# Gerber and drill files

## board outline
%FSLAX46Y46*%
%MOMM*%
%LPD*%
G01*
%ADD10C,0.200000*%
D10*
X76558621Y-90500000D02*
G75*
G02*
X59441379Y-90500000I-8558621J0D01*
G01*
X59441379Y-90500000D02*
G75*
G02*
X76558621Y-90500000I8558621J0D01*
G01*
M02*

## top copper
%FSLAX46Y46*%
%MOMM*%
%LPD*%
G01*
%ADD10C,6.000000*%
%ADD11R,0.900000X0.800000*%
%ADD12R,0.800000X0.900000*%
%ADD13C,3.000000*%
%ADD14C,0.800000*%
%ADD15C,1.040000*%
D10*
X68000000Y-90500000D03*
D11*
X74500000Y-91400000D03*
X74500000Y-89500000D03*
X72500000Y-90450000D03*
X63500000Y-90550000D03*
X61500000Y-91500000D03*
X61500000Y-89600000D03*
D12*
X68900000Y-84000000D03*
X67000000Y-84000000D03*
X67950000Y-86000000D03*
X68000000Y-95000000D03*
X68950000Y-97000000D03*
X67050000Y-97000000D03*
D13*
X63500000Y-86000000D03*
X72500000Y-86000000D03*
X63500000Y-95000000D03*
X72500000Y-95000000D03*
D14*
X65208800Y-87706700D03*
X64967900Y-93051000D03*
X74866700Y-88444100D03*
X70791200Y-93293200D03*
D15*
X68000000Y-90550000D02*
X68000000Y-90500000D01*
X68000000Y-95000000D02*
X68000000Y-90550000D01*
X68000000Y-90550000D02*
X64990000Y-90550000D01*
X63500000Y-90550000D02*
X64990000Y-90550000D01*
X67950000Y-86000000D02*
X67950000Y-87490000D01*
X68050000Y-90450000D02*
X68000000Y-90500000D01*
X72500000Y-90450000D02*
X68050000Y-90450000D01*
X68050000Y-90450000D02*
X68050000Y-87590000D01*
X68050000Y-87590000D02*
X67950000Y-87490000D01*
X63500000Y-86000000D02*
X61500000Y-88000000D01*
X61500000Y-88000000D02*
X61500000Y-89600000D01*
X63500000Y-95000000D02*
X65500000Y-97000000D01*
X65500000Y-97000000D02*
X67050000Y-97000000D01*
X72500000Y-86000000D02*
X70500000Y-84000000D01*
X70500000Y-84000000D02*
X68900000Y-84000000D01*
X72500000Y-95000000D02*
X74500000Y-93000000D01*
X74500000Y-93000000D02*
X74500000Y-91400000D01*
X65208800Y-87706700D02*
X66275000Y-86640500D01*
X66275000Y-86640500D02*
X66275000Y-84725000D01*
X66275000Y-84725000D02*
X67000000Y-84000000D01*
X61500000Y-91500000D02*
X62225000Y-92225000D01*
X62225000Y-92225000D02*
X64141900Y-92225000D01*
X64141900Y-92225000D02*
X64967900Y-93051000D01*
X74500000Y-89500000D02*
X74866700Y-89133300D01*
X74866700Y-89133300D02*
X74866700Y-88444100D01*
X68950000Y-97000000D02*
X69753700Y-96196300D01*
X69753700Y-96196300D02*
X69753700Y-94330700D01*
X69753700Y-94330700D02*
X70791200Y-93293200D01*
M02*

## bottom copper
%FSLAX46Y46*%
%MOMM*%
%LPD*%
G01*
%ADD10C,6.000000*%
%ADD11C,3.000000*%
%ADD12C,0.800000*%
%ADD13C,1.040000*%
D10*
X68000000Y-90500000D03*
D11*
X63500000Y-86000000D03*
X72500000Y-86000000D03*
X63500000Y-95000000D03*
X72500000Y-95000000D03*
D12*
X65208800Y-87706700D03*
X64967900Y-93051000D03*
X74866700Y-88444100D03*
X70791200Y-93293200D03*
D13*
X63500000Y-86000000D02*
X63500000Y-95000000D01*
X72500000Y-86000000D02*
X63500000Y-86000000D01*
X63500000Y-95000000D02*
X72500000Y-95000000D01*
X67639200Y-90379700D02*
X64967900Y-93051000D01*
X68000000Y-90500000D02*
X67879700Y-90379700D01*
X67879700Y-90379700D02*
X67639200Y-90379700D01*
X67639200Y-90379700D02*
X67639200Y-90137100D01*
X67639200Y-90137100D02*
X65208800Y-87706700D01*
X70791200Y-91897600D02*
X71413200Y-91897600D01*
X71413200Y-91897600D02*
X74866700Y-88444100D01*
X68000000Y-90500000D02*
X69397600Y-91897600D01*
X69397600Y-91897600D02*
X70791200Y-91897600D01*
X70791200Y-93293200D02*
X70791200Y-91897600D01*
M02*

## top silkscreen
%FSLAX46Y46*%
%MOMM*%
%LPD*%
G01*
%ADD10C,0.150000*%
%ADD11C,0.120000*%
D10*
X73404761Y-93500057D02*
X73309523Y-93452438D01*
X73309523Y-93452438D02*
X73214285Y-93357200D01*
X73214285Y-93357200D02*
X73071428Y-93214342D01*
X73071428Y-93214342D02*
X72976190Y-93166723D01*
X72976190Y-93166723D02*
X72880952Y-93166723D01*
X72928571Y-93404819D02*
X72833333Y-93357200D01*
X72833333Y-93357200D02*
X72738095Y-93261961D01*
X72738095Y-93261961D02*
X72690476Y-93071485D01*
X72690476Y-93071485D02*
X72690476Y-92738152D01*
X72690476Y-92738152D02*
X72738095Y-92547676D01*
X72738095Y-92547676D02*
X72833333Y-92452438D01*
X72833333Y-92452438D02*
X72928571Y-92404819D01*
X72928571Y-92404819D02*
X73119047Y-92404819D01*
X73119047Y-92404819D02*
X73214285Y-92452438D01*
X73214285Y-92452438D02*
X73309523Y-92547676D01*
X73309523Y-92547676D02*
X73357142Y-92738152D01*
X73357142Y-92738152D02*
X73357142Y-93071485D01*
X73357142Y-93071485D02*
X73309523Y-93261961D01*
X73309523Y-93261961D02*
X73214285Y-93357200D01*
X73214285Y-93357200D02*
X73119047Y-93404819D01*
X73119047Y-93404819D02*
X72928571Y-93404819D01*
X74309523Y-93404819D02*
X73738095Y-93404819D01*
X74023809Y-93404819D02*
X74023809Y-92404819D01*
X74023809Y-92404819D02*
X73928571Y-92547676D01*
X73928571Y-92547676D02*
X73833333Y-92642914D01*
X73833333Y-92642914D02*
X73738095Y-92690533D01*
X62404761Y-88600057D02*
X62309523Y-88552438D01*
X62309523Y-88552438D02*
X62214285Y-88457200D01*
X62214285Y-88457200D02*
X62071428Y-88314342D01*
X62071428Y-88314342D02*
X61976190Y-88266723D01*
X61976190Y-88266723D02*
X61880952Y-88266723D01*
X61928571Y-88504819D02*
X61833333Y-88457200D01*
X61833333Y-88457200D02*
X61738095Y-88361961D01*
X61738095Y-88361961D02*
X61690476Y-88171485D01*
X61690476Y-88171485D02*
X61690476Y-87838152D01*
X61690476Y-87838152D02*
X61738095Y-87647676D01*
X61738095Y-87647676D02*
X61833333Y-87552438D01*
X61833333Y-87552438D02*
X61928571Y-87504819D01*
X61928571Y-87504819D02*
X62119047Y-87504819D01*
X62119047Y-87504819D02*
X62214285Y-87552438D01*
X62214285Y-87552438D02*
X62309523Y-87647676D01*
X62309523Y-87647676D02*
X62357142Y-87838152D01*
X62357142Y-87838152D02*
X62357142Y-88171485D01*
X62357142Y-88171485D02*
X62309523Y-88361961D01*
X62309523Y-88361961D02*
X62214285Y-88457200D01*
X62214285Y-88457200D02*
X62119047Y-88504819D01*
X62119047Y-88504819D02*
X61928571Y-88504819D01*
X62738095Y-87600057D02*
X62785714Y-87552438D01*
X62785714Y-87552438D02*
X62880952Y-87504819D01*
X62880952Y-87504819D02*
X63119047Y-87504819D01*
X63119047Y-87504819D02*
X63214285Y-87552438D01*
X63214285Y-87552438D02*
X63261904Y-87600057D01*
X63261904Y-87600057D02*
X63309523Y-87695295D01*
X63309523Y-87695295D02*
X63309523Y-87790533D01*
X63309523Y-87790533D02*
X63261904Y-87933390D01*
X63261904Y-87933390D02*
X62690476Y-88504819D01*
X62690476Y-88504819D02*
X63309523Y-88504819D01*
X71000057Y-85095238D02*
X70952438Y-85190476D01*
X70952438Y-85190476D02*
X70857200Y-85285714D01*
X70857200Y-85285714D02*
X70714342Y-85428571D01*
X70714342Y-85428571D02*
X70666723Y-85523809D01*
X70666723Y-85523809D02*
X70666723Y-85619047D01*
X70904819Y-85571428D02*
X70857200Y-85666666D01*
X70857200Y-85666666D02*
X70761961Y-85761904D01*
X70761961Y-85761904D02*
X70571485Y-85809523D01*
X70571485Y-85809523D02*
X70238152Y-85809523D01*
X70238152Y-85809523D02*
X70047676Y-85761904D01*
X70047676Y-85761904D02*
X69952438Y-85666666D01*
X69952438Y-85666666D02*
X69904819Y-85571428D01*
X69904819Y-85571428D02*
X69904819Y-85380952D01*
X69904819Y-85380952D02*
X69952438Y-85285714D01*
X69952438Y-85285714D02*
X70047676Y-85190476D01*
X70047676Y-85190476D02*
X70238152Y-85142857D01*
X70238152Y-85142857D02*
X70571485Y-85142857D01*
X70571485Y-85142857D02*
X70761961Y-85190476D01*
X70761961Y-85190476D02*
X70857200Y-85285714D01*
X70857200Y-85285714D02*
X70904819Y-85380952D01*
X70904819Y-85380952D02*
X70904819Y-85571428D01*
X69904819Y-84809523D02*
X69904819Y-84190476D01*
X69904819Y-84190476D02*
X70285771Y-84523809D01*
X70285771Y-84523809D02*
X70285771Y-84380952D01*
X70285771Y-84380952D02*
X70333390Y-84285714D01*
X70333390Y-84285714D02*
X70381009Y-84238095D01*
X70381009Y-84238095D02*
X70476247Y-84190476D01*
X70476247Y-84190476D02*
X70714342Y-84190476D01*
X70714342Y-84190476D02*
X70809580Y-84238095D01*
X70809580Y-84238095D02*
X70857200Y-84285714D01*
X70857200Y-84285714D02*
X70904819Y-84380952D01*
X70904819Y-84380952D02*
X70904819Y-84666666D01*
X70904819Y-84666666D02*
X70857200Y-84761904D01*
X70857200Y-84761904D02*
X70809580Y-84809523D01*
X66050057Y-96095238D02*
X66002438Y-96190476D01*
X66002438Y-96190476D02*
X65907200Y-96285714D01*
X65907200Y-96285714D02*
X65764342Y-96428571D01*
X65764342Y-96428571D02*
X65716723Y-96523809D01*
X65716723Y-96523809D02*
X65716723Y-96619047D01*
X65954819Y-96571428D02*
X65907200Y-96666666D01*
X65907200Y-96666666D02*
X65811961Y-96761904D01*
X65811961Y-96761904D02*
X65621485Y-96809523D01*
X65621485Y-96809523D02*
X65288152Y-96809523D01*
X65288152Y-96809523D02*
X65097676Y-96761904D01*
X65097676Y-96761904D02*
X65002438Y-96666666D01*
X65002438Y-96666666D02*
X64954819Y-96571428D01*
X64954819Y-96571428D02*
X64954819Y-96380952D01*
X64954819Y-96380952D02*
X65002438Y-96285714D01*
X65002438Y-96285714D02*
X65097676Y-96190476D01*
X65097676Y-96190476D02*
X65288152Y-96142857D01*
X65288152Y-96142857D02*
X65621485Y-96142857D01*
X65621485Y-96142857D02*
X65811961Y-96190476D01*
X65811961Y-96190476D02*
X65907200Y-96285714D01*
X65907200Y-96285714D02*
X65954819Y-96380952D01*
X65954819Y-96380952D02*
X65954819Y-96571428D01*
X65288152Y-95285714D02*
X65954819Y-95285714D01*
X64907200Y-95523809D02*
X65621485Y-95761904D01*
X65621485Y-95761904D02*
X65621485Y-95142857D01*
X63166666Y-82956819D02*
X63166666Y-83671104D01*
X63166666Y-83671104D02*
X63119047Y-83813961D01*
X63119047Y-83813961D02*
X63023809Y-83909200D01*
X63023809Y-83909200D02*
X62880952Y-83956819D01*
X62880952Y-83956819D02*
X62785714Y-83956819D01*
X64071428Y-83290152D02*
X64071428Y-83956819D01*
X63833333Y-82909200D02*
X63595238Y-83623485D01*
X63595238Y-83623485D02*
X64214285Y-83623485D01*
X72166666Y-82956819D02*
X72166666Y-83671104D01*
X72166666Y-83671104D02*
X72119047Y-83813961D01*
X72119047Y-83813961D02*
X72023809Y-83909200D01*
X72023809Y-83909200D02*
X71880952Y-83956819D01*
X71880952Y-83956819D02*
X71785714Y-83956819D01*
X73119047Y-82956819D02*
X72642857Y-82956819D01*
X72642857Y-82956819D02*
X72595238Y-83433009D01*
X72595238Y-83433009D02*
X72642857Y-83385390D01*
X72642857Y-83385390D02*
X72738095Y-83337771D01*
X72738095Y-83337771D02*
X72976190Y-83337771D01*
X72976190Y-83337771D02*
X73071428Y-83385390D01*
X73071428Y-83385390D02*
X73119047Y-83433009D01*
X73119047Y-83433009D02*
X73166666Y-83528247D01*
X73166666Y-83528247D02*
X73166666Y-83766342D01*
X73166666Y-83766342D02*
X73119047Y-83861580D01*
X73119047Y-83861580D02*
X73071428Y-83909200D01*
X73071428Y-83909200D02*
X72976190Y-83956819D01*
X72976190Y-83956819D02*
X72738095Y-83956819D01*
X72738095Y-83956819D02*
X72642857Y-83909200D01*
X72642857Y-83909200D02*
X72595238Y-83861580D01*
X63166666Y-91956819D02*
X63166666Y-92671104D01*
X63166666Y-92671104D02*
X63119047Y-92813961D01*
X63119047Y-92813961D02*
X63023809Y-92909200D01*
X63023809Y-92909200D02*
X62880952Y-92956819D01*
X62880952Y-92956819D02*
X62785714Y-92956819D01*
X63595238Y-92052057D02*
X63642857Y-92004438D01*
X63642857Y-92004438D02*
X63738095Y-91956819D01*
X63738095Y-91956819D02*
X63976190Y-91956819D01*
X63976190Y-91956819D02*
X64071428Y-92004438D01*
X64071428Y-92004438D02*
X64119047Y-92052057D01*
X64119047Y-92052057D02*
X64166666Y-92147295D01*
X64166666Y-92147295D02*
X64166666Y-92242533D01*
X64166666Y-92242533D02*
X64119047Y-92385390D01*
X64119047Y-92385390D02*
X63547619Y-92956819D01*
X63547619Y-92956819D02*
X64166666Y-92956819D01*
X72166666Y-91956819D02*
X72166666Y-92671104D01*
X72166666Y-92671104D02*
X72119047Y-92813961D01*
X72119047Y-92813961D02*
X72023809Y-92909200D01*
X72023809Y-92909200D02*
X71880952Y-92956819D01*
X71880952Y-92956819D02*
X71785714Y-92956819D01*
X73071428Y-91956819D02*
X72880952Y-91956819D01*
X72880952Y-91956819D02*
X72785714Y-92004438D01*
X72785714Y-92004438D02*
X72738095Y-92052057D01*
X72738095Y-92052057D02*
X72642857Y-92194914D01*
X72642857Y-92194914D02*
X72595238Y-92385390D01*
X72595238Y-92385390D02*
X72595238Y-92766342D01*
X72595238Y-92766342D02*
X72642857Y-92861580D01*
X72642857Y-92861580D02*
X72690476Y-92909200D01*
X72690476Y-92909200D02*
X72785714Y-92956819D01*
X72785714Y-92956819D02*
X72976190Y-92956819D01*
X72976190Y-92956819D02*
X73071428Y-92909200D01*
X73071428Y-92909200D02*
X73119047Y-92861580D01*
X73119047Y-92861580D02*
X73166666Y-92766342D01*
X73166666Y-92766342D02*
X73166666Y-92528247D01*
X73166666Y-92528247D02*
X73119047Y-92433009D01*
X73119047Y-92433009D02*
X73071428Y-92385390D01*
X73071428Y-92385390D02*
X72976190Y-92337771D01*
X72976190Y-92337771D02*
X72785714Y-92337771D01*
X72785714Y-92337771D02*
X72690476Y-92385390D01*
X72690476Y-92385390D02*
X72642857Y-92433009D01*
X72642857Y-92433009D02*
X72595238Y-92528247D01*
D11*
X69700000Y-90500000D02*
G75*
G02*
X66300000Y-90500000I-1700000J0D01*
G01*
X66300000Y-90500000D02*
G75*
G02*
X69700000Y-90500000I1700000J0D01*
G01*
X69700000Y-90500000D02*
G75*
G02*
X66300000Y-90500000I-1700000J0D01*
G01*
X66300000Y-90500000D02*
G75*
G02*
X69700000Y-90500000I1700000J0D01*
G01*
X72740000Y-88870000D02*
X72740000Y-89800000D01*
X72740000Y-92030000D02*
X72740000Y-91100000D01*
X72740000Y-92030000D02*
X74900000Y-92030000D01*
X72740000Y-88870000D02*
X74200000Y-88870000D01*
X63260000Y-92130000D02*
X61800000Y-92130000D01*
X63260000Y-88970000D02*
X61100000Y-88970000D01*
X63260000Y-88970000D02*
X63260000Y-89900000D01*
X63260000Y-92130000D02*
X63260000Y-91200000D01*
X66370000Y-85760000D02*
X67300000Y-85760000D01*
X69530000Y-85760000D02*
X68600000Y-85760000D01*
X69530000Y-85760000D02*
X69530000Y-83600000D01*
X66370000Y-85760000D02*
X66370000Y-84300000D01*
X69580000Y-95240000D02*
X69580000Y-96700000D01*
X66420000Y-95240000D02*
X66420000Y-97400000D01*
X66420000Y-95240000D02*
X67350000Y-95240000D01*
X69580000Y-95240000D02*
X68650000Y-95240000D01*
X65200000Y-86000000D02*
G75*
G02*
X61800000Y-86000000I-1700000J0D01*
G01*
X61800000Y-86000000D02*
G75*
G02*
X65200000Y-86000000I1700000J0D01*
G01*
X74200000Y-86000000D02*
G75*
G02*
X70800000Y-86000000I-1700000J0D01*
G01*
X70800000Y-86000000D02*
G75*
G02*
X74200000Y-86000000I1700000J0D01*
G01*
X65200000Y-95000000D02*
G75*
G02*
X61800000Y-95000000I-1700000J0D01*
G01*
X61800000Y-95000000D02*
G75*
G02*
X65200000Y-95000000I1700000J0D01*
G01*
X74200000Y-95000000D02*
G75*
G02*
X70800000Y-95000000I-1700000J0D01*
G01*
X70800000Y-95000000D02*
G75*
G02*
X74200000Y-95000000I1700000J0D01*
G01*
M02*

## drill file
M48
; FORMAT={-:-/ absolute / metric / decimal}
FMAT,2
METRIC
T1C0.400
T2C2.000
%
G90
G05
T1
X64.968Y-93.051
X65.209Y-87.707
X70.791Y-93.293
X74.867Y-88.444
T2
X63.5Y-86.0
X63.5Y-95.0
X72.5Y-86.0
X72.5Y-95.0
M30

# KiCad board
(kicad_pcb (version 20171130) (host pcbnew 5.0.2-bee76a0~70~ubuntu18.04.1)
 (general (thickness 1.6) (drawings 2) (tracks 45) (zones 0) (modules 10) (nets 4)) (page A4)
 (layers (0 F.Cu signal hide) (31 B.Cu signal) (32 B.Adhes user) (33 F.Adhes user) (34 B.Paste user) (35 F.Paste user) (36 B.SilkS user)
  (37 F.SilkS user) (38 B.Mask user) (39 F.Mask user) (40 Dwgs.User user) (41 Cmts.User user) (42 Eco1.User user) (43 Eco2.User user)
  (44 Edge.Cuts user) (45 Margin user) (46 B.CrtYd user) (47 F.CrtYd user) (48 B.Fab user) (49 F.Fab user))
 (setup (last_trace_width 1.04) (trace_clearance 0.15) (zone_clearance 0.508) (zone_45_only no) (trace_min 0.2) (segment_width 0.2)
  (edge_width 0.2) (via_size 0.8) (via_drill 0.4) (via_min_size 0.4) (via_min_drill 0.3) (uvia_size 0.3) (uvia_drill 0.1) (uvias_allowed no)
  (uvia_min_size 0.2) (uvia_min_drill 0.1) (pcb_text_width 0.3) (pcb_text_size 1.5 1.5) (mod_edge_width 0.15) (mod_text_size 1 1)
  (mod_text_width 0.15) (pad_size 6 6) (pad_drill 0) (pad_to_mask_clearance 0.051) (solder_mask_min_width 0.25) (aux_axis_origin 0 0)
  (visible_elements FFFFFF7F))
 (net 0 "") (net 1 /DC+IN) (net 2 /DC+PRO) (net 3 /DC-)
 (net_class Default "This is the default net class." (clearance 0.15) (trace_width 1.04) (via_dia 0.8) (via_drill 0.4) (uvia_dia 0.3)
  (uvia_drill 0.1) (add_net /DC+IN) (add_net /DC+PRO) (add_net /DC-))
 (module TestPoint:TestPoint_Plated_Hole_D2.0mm (layer F.Cu) (at 68 90.5)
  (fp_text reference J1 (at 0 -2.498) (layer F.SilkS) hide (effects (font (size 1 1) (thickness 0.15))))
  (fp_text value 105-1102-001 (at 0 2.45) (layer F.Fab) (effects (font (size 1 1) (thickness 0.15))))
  (fp_circle (center 0 0) (end 0 -1.7) (layer F.SilkS) (width 0.12))
  (pad 1 smd circle (at 0 0) (size 6 6) (layers F.Cu F.Paste F.Mask) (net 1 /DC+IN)))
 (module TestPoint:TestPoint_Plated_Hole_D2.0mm (layer F.Cu) (at 68 90.5)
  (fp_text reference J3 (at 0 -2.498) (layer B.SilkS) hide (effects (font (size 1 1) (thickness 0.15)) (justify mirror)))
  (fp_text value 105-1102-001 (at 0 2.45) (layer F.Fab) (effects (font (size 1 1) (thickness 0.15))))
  (fp_circle (center 0 0) (end 0 -1.7) (layer F.SilkS) (width 0.12))
  (pad 1 smd circle (at 0 0) (size 6 6) (layers B.Cu F.Paste F.Mask) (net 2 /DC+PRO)))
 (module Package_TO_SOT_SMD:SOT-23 (layer F.Cu) (at 73.5 90.45 180)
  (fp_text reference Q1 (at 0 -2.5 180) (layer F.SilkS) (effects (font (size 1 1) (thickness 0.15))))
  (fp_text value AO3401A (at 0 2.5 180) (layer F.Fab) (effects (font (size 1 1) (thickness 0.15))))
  (fp_line (start 0.76 1.58) (end 0.76 0.65) (layer F.SilkS) (width 0.12))
  (fp_line (start 0.76 -1.58) (end 0.76 -0.65) (layer F.SilkS) (width 0.12))
  (fp_line (start 0.76 -1.58) (end -1.4 -1.58) (layer F.SilkS) (width 0.12))
  (fp_line (start 0.76 1.58) (end -0.7 1.58) (layer F.SilkS) (width 0.12))
  (pad 1 smd rect (at -1 -0.95 180) (size 0.9 0.8) (layers F.Cu F.Paste F.Mask) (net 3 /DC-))
  (pad 2 smd rect (at -1 0.95 180) (size 0.9 0.8) (layers F.Cu F.Paste F.Mask) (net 2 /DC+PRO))
  (pad 3 smd rect (at 1 0 180) (size 0.9 0.8) (layers F.Cu F.Paste F.Mask) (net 1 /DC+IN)))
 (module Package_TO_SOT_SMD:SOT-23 (layer F.Cu) (at 62.5 90.55)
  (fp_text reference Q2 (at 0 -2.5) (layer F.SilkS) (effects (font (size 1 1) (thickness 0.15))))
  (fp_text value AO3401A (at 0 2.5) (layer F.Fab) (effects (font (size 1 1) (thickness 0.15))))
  (fp_line (start 0.76 1.58) (end -0.7 1.58) (layer F.SilkS) (width 0.12))
  (fp_line (start 0.76 -1.58) (end -1.4 -1.58) (layer F.SilkS) (width 0.12))
  (fp_line (start 0.76 -1.58) (end 0.76 -0.65) (layer F.SilkS) (width 0.12))
  (fp_line (start 0.76 1.58) (end 0.76 0.65) (layer F.SilkS) (width 0.12))
  (pad 3 smd rect (at 1 0) (size 0.9 0.8) (layers F.Cu F.Paste F.Mask) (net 1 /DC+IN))
  (pad 2 smd rect (at -1 0.95) (size 0.9 0.8) (layers F.Cu F.Paste F.Mask) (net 2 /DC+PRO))
  (pad 1 smd rect (at -1 -0.95) (size 0.9 0.8) (layers F.Cu F.Paste F.Mask) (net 3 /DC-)))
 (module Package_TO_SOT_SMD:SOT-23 (layer F.Cu) (at 67.95 85 270)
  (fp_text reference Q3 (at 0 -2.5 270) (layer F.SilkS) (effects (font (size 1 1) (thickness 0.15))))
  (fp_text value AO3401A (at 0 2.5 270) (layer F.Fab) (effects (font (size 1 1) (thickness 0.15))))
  (fp_line (start 0.76 1.58) (end 0.76 0.65) (layer F.SilkS) (width 0.12))
  (fp_line (start 0.76 -1.58) (end 0.76 -0.65) (layer F.SilkS) (width 0.12))
  (fp_line (start 0.76 -1.58) (end -1.4 -1.58) (layer F.SilkS) (width 0.12))
  (fp_line (start 0.76 1.58) (end -0.7 1.58) (layer F.SilkS) (width 0.12))
  (pad 1 smd rect (at -1 -0.95 270) (size 0.9 0.8) (layers F.Cu F.Paste F.Mask) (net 3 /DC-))
  (pad 2 smd rect (at -1 0.95 270) (size 0.9 0.8) (layers F.Cu F.Paste F.Mask) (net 2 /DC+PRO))
  (pad 3 smd rect (at 1 0 270) (size 0.9 0.8) (layers F.Cu F.Paste F.Mask) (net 1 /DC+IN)))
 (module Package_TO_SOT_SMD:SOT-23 (layer F.Cu) (at 68 96 90)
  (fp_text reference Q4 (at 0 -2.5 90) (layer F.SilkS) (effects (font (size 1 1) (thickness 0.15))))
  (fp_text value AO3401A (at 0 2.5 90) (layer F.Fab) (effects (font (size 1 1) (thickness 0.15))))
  (fp_line (start 0.76 1.58) (end -0.7 1.58) (layer F.SilkS) (width 0.12))
  (fp_line (start 0.76 -1.58) (end -1.4 -1.58) (layer F.SilkS) (width 0.12))
  (fp_line (start 0.76 -1.58) (end 0.76 -0.65) (layer F.SilkS) (width 0.12))
  (fp_line (start 0.76 1.58) (end 0.76 0.65) (layer F.SilkS) (width 0.12))
  (pad 3 smd rect (at 1 0 90) (size 0.9 0.8) (layers F.Cu F.Paste F.Mask) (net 1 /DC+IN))
  (pad 2 smd rect (at -1 0.95 90) (size 0.9 0.8) (layers F.Cu F.Paste F.Mask) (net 2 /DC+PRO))
  (pad 1 smd rect (at -1 -0.95 90) (size 0.9 0.8) (layers F.Cu F.Paste F.Mask) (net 3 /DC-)))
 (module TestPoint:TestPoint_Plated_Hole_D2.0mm (layer F.Cu) (at 63.5 86)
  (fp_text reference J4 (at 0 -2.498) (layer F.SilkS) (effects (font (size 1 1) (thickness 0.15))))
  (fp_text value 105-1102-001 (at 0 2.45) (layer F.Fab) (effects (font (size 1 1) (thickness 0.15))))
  (fp_circle (center 0 0) (end 0 -1.7) (layer F.SilkS) (width 0.12))
  (pad 1 thru_hole circle (at 0 0) (size 3 3) (drill 2) (layers *.Cu *.Mask) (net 3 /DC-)))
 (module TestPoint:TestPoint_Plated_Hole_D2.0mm (layer F.Cu) (at 72.5 86)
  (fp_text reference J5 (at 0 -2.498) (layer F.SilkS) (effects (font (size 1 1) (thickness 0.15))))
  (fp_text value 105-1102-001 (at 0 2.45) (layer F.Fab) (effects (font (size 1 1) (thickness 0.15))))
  (fp_circle (center 0 0) (end 0 -1.7) (layer F.SilkS) (width 0.12))
  (pad 1 thru_hole circle (at 0 0) (size 3 3) (drill 2) (layers *.Cu *.Mask) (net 3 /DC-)))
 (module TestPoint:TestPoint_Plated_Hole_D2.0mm (layer F.Cu) (at 63.5 95)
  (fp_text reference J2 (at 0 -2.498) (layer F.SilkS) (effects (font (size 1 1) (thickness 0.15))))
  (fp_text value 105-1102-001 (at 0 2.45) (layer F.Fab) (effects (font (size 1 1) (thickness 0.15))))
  (fp_circle (center 0 0) (end 0 -1.7) (layer F.SilkS) (width 0.12))
  (pad 1 thru_hole circle (at 0 0) (size 3 3) (drill 2) (layers *.Cu *.Mask) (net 3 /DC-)))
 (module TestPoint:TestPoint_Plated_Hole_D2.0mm (layer F.Cu) (at 72.5 95)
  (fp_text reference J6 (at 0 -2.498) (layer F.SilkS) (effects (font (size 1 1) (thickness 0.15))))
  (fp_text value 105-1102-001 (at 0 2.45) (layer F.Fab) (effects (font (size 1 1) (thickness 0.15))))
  (fp_circle (center 0 0) (end 0 -1.7) (layer F.SilkS) (width 0.12))
  (pad 1 thru_hole circle (at 0 0) (size 3 3) (drill 2) (layers *.Cu *.Mask) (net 3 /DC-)))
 (gr_circle (center 68 90.5) (end 76.558621 90.5) (layer Edge.Cuts) (width 0.2))
 (segment (start 68 90.55) (end 68 90.5) (width 1.04) (layer F.Cu) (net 1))
 (segment (start 68 95) (end 68 90.55) (width 1.04) (layer F.Cu) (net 1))
 (segment (start 68 90.55) (end 64.99 90.55) (width 1.04) (layer F.Cu) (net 1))
 (segment (start 63.5 90.55) (end 64.99 90.55) (width 1.04) (layer F.Cu) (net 1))
 (segment (start 67.95 86) (end 67.95 87.49) (width 1.04) (layer F.Cu) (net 1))
 (segment (start 68.05 90.45) (end 68 90.5) (width 1.04) (layer F.Cu) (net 1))
 (segment (start 72.5 90.45) (end 68.05 90.45) (width 1.04) (layer F.Cu) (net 1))
 (segment (start 68.05 90.45) (end 68.05 87.59) (width 1.04) (layer F.Cu) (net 1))
 (segment (start 68.05 87.59) (end 67.95 87.49) (width 1.04) (layer F.Cu) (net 1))
 (segment (start 63.5 86) (end 63.5 95) (width 1.04) (layer B.Cu) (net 3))
 (segment (start 72.5 86) (end 63.5 86) (width 1.04) (layer B.Cu) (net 3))
 (segment (start 63.5 95) (end 72.5 95) (width 1.04) (layer B.Cu) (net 3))
 (segment (start 63.5 86) (end 61.5 88) (width 1.04) (layer F.Cu) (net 3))
 (segment (start 61.5 88) (end 61.5 89.6) (width 1.04) (layer F.Cu) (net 3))
 (segment (start 63.5 95) (end 65.5 97) (width 1.04) (layer F.Cu) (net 3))
 (segment (start 65.5 97) (end 67.05 97) (width 1.04) (layer F.Cu) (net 3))
 (segment (start 72.5 86) (end 70.5 84) (width 1.04) (layer F.Cu) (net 3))
 (segment (start 70.5 84) (end 68.9 84) (width 1.04) (layer F.Cu) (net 3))
 (segment (start 72.5 95) (end 74.5 93) (width 1.04) (layer F.Cu) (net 3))
 (segment (start 74.5 93) (end 74.5 91.4) (width 1.04) (layer F.Cu) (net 3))
 (segment (start 67.6392 90.3797) (end 64.9679 93.051) (width 1.04) (layer B.Cu) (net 2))
 (segment (start 68 90.5) (end 67.8797 90.3797) (width 1.04) (layer B.Cu) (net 2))
 (segment (start 67.8797 90.3797) (end 67.6392 90.3797) (width 1.04) (layer B.Cu) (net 2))
 (segment (start 67.6392 90.3797) (end 67.6392 90.1371) (width 1.04) (layer B.Cu) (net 2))
 (segment (start 67.6392 90.1371) (end 65.2088 87.7067) (width 1.04) (layer B.Cu) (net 2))
 (segment (start 65.2088 87.7067) (end 66.275 86.6405) (width 1.04) (layer F.Cu) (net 2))
 (segment (start 66.275 86.6405) (end 66.275 84.725) (width 1.04) (layer F.Cu) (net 2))
 (segment (start 66.275 84.725) (end 67 84) (width 1.04) (layer F.Cu) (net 2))
 (segment (start 61.5 91.5) (end 62.225 92.225) (width 1.04) (layer F.Cu) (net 2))
 (segment (start 62.225 92.225) (end 64.1419 92.225) (width 1.04) (layer F.Cu) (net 2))
 (segment (start 64.1419 92.225) (end 64.9679 93.051) (width 1.04) (layer F.Cu) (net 2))
 (segment (start 70.7912 91.8976) (end 71.4132 91.8976) (width 1.04) (layer B.Cu) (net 2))
 (segment (start 71.4132 91.8976) (end 74.8667 88.4441) (width 1.04) (layer B.Cu) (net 2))
 (segment (start 68 90.5) (end 69.3976 91.8976) (width 1.04) (layer B.Cu) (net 2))
 (segment (start 69.3976 91.8976) (end 70.7912 91.8976) (width 1.04) (layer B.Cu) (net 2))
 (segment (start 70.7912 93.2932) (end 70.7912 91.8976) (width 1.04) (layer B.Cu) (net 2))
 (segment (start 74.5 89.5) (end 74.8667 89.1333) (width 1.04) (layer F.Cu) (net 2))
 (segment (start 74.8667 89.1333) (end 74.8667 88.4441) (width 1.04) (layer F.Cu) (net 2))
 (segment (start 68.95 97) (end 69.7537 96.1963) (width 1.04) (layer F.Cu) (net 2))
 (segment (start 69.7537 96.1963) (end 69.7537 94.3307) (width 1.04) (layer F.Cu) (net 2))
 (segment (start 69.7537 94.3307) (end 70.7912 93.2932) (width 1.04) (layer F.Cu) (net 2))
 (via (at 65.2088 87.7067) (size 0.8) (layers F.Cu B.Cu) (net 2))
 (via (at 64.9679 93.051) (size 0.8) (layers F.Cu B.Cu) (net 2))
 (via (at 74.8667 88.4441) (size 0.8) (layers F.Cu B.Cu) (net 2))
 (via (at 70.7912 93.2932) (size 0.8) (layers F.Cu B.Cu) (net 2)))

